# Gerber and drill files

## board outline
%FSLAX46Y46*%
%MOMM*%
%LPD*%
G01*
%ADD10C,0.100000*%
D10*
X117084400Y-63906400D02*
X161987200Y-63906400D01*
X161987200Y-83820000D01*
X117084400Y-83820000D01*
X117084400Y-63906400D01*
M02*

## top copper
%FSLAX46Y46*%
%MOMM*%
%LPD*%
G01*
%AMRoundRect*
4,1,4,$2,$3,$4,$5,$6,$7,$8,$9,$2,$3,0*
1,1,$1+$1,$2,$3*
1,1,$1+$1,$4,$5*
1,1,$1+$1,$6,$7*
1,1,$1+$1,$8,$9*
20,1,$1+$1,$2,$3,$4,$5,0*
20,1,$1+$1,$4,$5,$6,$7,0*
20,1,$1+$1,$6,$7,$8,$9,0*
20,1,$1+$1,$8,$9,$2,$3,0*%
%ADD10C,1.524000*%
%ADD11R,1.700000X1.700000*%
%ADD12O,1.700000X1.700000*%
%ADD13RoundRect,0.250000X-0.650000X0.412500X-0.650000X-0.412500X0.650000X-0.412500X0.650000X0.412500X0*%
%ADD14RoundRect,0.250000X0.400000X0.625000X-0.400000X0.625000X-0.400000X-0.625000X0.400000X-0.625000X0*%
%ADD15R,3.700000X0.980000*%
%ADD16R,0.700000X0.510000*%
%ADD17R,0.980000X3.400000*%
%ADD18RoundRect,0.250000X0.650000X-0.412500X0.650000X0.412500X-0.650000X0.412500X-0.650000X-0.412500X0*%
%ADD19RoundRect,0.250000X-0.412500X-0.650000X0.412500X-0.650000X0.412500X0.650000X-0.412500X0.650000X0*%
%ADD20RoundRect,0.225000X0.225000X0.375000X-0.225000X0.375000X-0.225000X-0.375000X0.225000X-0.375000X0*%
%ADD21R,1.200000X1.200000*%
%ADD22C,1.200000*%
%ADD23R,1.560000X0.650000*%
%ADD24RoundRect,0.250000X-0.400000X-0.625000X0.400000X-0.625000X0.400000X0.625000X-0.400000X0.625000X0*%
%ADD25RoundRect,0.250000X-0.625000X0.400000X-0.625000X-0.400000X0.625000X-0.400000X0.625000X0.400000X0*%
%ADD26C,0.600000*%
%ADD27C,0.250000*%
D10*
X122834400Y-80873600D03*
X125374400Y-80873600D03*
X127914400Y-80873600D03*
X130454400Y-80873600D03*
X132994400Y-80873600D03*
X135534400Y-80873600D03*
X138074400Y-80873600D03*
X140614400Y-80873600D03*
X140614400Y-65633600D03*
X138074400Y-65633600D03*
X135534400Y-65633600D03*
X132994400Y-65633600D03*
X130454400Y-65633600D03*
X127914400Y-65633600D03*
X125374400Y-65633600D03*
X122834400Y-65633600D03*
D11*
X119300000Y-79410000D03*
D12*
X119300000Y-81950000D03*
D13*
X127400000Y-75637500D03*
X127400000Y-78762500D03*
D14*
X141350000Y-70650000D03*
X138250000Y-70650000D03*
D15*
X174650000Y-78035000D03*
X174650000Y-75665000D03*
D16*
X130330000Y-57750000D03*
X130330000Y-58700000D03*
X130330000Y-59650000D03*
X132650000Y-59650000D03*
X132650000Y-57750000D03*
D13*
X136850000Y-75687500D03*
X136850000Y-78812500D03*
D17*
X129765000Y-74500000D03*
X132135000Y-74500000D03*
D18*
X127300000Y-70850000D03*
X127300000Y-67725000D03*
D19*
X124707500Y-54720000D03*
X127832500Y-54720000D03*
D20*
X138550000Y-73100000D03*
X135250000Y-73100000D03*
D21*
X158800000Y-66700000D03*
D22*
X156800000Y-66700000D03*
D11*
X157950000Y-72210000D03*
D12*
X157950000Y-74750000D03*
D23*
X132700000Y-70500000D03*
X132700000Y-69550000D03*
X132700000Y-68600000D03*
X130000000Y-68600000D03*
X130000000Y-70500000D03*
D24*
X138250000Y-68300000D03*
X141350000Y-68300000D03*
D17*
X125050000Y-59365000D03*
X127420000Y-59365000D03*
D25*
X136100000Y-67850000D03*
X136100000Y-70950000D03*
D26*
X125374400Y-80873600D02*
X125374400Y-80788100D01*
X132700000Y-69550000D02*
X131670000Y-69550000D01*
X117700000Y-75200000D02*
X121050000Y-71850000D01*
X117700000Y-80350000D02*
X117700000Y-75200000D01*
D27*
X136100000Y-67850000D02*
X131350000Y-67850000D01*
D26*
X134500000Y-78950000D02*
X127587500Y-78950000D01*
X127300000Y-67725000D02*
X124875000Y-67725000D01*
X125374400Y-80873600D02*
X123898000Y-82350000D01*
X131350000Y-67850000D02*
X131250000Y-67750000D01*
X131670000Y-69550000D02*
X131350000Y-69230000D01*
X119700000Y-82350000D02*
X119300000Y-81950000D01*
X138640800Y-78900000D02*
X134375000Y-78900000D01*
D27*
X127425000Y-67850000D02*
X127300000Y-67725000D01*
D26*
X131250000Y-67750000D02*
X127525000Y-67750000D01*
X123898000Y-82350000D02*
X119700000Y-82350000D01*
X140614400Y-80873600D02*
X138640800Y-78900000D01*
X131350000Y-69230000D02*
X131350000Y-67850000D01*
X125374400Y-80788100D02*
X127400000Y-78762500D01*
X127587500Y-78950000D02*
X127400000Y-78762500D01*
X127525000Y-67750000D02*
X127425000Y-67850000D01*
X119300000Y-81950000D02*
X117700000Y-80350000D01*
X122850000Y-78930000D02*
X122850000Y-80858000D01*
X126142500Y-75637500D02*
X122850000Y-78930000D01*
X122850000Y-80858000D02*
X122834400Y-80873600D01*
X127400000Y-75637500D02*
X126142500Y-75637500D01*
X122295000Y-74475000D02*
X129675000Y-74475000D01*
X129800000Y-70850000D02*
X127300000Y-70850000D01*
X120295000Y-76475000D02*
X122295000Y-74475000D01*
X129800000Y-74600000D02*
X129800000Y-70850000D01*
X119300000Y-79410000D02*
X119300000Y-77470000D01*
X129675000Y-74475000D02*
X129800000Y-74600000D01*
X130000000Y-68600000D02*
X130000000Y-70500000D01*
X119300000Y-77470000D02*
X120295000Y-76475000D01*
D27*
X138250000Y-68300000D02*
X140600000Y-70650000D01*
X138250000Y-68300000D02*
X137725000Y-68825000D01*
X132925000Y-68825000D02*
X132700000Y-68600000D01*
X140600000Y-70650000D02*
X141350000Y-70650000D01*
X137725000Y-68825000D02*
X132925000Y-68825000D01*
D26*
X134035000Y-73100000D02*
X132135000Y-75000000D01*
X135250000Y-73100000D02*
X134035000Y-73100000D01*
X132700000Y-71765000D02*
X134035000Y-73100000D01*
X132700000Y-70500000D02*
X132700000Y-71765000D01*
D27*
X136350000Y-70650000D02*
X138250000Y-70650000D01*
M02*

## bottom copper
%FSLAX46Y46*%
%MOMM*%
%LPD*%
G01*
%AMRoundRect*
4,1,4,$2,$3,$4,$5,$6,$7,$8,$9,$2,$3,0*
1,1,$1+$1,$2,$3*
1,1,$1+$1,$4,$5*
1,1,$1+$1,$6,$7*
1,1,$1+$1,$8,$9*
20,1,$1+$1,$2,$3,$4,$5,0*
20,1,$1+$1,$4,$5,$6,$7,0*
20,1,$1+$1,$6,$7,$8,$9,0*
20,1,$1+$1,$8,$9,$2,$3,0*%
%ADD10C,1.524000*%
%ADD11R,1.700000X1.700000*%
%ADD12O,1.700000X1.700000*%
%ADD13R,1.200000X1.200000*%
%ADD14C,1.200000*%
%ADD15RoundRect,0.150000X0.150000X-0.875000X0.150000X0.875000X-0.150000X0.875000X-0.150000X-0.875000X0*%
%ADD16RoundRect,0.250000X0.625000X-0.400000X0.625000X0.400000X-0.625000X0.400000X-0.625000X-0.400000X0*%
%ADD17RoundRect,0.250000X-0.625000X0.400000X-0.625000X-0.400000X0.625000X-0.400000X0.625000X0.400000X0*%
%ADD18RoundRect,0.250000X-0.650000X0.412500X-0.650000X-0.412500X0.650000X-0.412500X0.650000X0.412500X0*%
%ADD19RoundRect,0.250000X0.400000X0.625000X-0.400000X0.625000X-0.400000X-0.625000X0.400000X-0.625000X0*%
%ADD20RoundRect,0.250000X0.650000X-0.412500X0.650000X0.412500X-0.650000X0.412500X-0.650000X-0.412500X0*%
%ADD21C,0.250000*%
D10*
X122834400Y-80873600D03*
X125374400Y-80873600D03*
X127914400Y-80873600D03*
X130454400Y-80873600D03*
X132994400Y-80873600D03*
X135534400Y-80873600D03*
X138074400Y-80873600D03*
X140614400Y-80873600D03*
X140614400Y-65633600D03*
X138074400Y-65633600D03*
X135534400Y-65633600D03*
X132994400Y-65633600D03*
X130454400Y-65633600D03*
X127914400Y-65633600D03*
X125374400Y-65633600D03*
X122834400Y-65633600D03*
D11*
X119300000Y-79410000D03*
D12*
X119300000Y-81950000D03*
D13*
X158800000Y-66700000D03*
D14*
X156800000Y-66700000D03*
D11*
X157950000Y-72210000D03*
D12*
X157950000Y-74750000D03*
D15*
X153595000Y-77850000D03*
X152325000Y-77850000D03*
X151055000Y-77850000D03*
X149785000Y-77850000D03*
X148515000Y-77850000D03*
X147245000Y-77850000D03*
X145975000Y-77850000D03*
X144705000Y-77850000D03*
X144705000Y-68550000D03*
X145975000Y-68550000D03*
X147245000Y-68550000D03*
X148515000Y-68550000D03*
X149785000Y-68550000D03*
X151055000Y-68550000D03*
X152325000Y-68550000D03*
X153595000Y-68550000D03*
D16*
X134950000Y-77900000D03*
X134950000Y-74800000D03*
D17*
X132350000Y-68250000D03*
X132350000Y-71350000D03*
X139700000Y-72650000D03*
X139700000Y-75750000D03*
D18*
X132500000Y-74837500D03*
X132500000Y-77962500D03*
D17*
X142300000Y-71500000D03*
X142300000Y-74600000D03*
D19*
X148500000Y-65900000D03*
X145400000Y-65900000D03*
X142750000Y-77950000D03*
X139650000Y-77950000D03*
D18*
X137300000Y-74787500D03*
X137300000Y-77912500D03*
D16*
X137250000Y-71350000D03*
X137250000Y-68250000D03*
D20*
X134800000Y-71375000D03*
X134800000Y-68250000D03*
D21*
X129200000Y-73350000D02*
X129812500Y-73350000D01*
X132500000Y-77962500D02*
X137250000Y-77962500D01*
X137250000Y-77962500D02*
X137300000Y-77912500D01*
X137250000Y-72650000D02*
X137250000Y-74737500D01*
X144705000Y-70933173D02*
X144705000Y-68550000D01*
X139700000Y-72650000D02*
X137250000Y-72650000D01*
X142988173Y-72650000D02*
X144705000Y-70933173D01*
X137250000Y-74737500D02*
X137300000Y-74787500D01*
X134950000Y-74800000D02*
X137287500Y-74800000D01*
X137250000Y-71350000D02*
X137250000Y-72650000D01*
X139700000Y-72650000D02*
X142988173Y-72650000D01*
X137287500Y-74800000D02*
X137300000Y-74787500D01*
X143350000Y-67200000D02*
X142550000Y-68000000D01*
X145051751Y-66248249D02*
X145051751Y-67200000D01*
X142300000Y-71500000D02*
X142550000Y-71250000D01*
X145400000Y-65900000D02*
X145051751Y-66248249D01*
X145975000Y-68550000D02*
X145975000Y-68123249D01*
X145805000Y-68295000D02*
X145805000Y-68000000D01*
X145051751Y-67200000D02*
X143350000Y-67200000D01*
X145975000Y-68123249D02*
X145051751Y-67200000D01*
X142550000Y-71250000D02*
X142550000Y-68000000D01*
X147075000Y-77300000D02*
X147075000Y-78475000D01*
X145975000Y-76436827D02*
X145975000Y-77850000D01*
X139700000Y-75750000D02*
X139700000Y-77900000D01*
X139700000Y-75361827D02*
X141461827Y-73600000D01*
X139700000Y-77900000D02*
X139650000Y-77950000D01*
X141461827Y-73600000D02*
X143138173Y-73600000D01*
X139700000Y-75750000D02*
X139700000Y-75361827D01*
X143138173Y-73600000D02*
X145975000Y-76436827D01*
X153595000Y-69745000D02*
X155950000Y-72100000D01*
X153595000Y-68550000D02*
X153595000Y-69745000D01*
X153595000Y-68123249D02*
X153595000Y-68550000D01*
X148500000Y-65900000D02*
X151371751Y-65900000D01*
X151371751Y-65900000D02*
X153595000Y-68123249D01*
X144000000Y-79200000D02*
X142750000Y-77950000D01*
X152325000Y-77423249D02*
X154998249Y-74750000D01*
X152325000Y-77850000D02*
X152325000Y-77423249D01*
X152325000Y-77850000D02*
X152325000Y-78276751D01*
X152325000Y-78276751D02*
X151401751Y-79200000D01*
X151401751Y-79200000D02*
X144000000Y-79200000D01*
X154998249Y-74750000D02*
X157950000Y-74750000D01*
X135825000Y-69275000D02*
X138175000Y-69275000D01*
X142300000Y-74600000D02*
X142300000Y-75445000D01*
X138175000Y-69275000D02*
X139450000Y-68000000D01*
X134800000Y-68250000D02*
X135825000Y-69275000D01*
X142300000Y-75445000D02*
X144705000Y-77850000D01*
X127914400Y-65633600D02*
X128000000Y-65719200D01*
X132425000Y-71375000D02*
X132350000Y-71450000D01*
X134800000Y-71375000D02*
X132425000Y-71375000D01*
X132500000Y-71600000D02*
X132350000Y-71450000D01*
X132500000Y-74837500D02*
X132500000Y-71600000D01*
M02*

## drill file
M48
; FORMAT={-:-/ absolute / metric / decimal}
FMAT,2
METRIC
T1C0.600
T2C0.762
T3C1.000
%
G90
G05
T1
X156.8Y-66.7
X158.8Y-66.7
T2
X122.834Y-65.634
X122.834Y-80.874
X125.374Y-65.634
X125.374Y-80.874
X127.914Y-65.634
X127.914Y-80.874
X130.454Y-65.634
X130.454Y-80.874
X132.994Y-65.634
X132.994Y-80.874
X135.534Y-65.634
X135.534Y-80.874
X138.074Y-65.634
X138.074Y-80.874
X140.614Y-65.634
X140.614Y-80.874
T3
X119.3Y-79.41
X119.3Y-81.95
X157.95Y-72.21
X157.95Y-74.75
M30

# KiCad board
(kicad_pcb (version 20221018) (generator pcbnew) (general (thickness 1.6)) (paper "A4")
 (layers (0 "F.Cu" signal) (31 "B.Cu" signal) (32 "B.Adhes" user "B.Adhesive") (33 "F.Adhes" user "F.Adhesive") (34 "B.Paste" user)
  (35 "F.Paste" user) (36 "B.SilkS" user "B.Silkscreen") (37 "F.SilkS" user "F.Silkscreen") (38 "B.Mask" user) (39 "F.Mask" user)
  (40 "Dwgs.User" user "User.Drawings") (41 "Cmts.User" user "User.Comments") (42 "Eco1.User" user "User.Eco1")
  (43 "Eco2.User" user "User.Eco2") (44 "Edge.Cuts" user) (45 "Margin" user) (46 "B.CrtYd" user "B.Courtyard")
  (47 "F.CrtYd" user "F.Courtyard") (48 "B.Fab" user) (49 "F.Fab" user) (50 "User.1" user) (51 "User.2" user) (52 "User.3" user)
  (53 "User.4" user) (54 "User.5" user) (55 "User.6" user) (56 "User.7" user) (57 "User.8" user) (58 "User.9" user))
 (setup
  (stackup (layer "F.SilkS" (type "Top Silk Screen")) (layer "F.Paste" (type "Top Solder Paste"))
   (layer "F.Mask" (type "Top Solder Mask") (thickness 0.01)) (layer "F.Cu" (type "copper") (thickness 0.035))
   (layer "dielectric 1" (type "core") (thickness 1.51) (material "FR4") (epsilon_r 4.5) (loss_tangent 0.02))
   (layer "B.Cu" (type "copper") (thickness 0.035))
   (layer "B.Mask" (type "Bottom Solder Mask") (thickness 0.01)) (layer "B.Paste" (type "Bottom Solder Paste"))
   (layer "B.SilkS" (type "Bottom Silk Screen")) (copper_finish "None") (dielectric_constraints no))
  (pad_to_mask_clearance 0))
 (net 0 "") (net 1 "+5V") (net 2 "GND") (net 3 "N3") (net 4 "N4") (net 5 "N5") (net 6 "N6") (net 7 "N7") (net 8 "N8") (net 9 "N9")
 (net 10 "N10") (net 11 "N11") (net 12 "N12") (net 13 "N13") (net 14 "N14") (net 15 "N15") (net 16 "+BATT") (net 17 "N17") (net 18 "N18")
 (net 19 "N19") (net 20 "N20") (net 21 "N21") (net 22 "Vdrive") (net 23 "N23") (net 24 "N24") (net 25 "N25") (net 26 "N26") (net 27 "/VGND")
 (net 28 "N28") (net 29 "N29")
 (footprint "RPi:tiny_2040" (layer "F.Cu") (at 130.4544 73.2536 90)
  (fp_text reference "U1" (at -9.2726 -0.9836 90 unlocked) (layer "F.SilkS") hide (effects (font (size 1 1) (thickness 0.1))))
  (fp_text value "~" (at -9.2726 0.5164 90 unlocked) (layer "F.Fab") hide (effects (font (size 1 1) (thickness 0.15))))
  (pad "1" thru_hole circle (at -7.62 -7.62 90) (size 1.524 1.524) (drill 0.762) (layers "*.Cu" "*.Mask") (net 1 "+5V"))
  (pad "2" thru_hole circle (at -7.62 -5.08 90) (size 1.524 1.524) (drill 0.762) (layers "*.Cu" "*.Mask") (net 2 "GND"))
  (pad "3" thru_hole circle (at -7.62 -2.54 90) (size 1.524 1.524) (drill 0.762) (layers "*.Cu" "*.Mask") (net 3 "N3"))
  (pad "4" thru_hole circle (at -7.62 0 90) (size 1.524 1.524) (drill 0.762) (layers "*.Cu" "*.Mask") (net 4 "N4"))
  (pad "5" thru_hole circle (at -7.62 2.54 90) (size 1.524 1.524) (drill 0.762) (layers "*.Cu" "*.Mask") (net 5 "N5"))
  (pad "6" thru_hole circle (at -7.62 5.08 90) (size 1.524 1.524) (drill 0.762) (layers "*.Cu" "*.Mask") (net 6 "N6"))
  (pad "7" thru_hole circle (at -7.62 7.62 90) (size 1.524 1.524) (drill 0.762) (layers "*.Cu" "*.Mask") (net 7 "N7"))
  (pad "8" thru_hole circle (at -7.62 10.16 90) (size 1.524 1.524) (drill 0.762) (layers "*.Cu" "*.Mask") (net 2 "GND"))
  (pad "9" thru_hole circle (at 7.62 10.16 90) (size 1.524 1.524) (drill 0.762) (layers "*.Cu" "*.Mask") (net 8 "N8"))
  (pad "10" thru_hole circle (at 7.62 7.62 90) (size 1.524 1.524) (drill 0.762) (layers "*.Cu" "*.Mask") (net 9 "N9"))
  (pad "11" thru_hole circle (at 7.62 5.08 90) (size 1.524 1.524) (drill 0.762) (layers "*.Cu" "*.Mask") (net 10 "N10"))
  (pad "12" thru_hole circle (at 7.62 2.54 90) (size 1.524 1.524) (drill 0.762) (layers "*.Cu" "*.Mask") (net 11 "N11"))
  (pad "13" thru_hole circle (at 7.62 0 90) (size 1.524 1.524) (drill 0.762) (layers "*.Cu" "*.Mask") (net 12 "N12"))
  (pad "14" thru_hole circle (at 7.62 -2.54 90) (size 1.524 1.524) (drill 0.762) (layers "*.Cu" "*.Mask") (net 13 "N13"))
  (pad "15" thru_hole circle (at 7.62 -5.08 90) (size 1.524 1.524) (drill 0.762) (layers "*.Cu" "*.Mask") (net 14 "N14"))
  (pad "16" thru_hole circle (at 7.62 -7.62 90) (size 1.524 1.524) (drill 0.762) (layers "*.Cu" "*.Mask") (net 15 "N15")))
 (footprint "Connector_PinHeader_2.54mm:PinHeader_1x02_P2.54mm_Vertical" (layer "F.Cu") (at 119.3 79.41)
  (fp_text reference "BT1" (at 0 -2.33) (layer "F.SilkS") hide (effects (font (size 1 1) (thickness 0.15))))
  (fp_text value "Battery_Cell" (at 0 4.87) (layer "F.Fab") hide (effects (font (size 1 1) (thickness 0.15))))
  (pad "1" thru_hole rect (at 0 0) (size 1.7 1.7) (drill 1) (layers "*.Cu" "*.Mask") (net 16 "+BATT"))
  (pad "2" thru_hole oval (at 0 2.54) (size 1.7 1.7) (drill 1) (layers "*.Cu" "*.Mask") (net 2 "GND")))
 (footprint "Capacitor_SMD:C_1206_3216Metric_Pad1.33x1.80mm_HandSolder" (layer "F.Cu") (at 127.4 77.2 -90)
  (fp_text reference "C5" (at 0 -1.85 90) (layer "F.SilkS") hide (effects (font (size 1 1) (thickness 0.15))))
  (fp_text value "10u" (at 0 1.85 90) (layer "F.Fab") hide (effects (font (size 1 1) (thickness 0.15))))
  (pad "1" smd roundrect (at -1.5625 0 270) (size 1.325 1.8) (layers "F.Cu" "F.Paste" "F.Mask") (roundrect_rratio 0.188679) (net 1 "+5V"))
  (pad "2" smd roundrect (at 1.5625 0 270) (size 1.325 1.8) (layers "F.Cu" "F.Paste" "F.Mask") (roundrect_rratio 0.188679) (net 2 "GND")))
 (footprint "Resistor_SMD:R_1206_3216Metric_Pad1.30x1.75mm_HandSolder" (layer "F.Cu") (at 139.8 70.65 180)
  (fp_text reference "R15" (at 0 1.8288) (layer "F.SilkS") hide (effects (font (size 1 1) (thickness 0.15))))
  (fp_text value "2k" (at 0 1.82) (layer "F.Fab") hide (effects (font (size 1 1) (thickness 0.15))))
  (pad "1" smd roundrect (at -1.55 0 180) (size 1.3 1.75) (layers "F.Cu" "F.Paste" "F.Mask") (roundrect_rratio 0.1923076923) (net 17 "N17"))
  (pad "2" smd roundrect (at 1.55 0 180) (size 1.3 1.75) (layers "F.Cu" "F.Paste" "F.Mask") (roundrect_rratio 0.1923076923) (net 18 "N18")))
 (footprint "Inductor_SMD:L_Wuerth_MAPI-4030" (layer "F.Cu") (at 174.65 76.85 90)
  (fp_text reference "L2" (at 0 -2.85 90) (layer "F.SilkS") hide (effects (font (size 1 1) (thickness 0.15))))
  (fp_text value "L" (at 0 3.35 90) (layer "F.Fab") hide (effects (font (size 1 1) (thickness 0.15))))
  (pad "1" smd rect (at -1.185 0 90) (size 0.98 3.7) (layers "F.Cu" "F.Paste" "F.Mask") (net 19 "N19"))
  (pad "2" smd rect (at 1.185 0 90) (size 0.98 3.7) (layers "F.Cu" "F.Paste" "F.Mask") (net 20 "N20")))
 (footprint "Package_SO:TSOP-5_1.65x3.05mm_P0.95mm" (layer "F.Cu") (at 131.49 58.7)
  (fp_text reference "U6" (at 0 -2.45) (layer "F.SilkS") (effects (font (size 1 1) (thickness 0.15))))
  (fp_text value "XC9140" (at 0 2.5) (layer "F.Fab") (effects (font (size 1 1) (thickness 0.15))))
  (pad "1" smd rect (at -1.16 -0.95) (size 0.7 0.51) (layers "F.Cu" "F.Paste" "F.Mask") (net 16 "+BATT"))
  (pad "2" smd rect (at -1.16 0) (size 0.7 0.51) (layers "F.Cu" "F.Paste" "F.Mask") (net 2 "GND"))
  (pad "3" smd rect (at -1.16 0.95) (size 0.7 0.51) (layers "F.Cu" "F.Paste" "F.Mask") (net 16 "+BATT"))
  (pad "4" smd rect (at 1.16 0.95) (size 0.7 0.51) (layers "F.Cu" "F.Paste" "F.Mask") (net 1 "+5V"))
  (pad "5" smd rect (at 1.16 -0.95) (size 0.7 0.51) (layers "F.Cu" "F.Paste" "F.Mask") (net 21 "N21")))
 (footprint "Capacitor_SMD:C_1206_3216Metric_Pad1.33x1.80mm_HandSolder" (layer "F.Cu") (at 136.85 77.25 -90)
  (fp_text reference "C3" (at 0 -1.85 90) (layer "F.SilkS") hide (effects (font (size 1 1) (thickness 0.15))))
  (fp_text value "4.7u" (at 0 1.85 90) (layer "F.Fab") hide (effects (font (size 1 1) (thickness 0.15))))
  (pad "1" smd roundrect (at -1.5625 0 270) (size 1.325 1.8) (layers "F.Cu" "F.Paste" "F.Mask") (roundrect_rratio 0.1886792453)
   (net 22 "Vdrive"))
  (pad "2" smd roundrect (at 1.5625 0 270) (size 1.325 1.8) (layers "F.Cu" "F.Paste" "F.Mask") (roundrect_rratio 0.1886792453) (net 2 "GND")))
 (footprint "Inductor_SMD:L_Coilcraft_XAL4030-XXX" (layer "F.Cu") (at 130.95 74.5)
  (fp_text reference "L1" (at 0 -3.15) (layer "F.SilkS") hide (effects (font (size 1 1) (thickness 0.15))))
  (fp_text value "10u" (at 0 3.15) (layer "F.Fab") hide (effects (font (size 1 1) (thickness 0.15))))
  (pad "1" smd rect (at -1.185 0) (size 0.98 3.4) (layers "F.Cu" "F.Paste" "F.Mask") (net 16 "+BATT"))
  (pad "2" smd rect (at 1.185 0) (size 0.98 3.4) (layers "F.Cu" "F.Paste" "F.Mask") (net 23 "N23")))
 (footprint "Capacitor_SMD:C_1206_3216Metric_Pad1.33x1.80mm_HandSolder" (layer "F.Cu") (at 127.3 69.2875 90)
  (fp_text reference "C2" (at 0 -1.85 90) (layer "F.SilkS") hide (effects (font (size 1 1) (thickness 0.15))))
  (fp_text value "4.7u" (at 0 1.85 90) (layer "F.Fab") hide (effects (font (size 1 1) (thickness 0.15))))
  (pad "1" smd roundrect (at -1.5625 0 90) (size 1.325 1.8) (layers "F.Cu" "F.Paste" "F.Mask") (roundrect_rratio 0.188679) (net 16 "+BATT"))
  (pad "2" smd roundrect (at 1.5625 0 90) (size 1.325 1.8) (layers "F.Cu" "F.Paste" "F.Mask") (roundrect_rratio 0.188679) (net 2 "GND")))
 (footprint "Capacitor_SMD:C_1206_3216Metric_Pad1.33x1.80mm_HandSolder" (layer "F.Cu") (at 126.27 54.72)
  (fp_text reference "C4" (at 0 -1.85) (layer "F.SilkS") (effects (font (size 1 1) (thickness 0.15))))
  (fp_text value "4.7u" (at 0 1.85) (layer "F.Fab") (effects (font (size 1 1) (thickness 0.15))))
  (pad "1" smd roundrect (at -1.5625 0) (size 1.325 1.8) (layers "F.Cu" "F.Paste" "F.Mask") (roundrect_rratio 0.188679) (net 16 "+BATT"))
  (pad "2" smd roundrect (at 1.5625 0) (size 1.325 1.8) (layers "F.Cu" "F.Paste" "F.Mask") (roundrect_rratio 0.188679) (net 2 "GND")))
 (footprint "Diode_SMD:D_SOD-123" (layer "F.Cu") (at 136.9 73.1 180)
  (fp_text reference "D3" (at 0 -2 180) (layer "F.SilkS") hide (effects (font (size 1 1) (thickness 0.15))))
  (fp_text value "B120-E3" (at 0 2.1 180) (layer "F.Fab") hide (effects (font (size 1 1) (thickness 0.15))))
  (pad "1" smd roundrect (at -1.65 0 180) (size 0.9 1.2) (layers "F.Cu" "F.Paste" "F.Mask") (roundrect_rratio 0.25) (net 22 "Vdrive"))
  (pad "2" smd roundrect (at 1.65 0 180) (size 0.9 1.2) (layers "F.Cu" "F.Paste" "F.Mask") (roundrect_rratio 0.25) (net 23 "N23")))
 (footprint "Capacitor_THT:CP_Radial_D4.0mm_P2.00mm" (layer "F.Cu") (at 158.8 66.7 180)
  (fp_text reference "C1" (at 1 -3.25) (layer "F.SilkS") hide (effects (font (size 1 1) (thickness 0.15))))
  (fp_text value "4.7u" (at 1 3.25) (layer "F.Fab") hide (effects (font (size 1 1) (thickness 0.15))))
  (pad "1" thru_hole rect (at 0 0 180) (size 1.2 1.2) (drill 0.6) (layers "*.Cu" "*.Mask") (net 22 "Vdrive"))
  (pad "2" thru_hole circle (at 2 0 180) (size 1.2 1.2) (drill 0.6) (layers "*.Cu" "*.Mask") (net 2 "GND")))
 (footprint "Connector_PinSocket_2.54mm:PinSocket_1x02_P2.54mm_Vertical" (layer "F.Cu") (at 157.95 72.21)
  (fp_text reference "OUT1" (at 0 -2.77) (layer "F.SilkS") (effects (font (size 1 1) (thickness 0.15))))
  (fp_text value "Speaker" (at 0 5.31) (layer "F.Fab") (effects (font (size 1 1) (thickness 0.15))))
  (pad "1" thru_hole rect (at 0 0) (size 1.7 1.7) (drill 1) (layers "*.Cu" "*.Mask") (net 20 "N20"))
  (pad "2" thru_hole oval (at 0 2.54) (size 1.7 1.7) (drill 1) (layers "*.Cu" "*.Mask") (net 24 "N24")))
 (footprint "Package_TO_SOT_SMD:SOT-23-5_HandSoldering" (layer "F.Cu") (at 131.35 69.55 180)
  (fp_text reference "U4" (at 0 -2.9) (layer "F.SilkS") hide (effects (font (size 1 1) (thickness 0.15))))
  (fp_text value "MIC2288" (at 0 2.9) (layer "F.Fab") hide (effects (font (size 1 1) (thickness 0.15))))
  (pad "1" smd rect (at -1.35 -0.95 180) (size 1.56 0.65) (layers "F.Cu" "F.Paste" "F.Mask") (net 23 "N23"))
  (pad "2" smd rect (at -1.35 0 180) (size 1.56 0.65) (layers "F.Cu" "F.Paste" "F.Mask") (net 2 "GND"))
  (pad "3" smd rect (at -1.35 0.95 180) (size 1.56 0.65) (layers "F.Cu" "F.Paste" "F.Mask") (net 17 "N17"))
  (pad "4" smd rect (at 1.35 0.95 180) (size 1.56 0.65) (layers "F.Cu" "F.Paste" "F.Mask") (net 16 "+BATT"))
  (pad "5" smd rect (at 1.35 -0.95 180) (size 1.56 0.65) (layers "F.Cu" "F.Paste" "F.Mask") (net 16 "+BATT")))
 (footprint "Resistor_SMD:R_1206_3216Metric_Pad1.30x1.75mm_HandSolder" (layer "F.Cu") (at 139.8 68.3)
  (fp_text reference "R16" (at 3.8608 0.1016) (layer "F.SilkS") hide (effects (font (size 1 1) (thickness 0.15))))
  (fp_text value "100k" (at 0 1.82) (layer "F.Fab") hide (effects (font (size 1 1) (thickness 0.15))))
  (pad "1" smd roundrect (at -1.55 0) (size 1.3 1.75) (layers "F.Cu" "F.Paste" "F.Mask") (roundrect_rratio 0.1923076923) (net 17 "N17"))
  (pad "2" smd roundrect (at 1.55 0) (size 1.3 1.75) (layers "F.Cu" "F.Paste" "F.Mask") (roundrect_rratio 0.1923076923) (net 22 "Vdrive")))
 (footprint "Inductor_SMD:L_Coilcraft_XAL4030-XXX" (layer "F.Cu") (at 126.235 59.365)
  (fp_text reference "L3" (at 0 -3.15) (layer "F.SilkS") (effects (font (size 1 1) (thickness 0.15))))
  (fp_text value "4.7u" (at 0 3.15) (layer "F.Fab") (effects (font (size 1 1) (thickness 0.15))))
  (pad "1" smd rect (at -1.185 0) (size 0.98 3.4) (layers "F.Cu" "F.Paste" "F.Mask") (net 16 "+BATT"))
  (pad "2" smd rect (at 1.185 0) (size 0.98 3.4) (layers "F.Cu" "F.Paste" "F.Mask") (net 21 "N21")))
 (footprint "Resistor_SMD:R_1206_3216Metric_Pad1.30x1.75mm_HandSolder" (layer "F.Cu") (at 136.1 69.4 -90)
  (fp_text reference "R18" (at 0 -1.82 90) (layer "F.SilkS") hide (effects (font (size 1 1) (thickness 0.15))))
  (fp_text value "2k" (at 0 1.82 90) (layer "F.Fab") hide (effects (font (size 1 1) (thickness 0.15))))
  (pad "1" smd roundrect (at -1.55 0 270) (size 1.3 1.75) (layers "F.Cu" "F.Paste" "F.Mask") (roundrect_rratio 0.1923076923) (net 2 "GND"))
  (pad "2" smd roundrect (at 1.55 0 270) (size 1.3 1.75) (layers "F.Cu" "F.Paste" "F.Mask") (roundrect_rratio 0.1923076923) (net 18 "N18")))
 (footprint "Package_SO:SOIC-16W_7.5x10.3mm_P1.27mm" (layer "B.Cu") (at 149.15 73.2 90)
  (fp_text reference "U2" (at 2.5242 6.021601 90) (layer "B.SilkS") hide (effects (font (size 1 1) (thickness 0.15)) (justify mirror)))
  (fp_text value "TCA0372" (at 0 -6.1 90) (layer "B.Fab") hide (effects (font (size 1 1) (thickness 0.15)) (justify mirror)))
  (pad "1" smd roundrect (at -4.65 4.445 90) (size 2.05 0.6) (layers "B.Cu" "B.Paste" "B.Mask") (roundrect_rratio 0.25) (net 22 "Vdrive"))
  (pad "2" smd roundrect (at -4.65 3.175 90) (size 2.05 0.6) (layers "B.Cu" "B.Paste" "B.Mask") (roundrect_rratio 0.25) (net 24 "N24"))
  (pad "3" smd roundrect (at -4.65 1.905 90) (size 2.05 0.6) (layers "B.Cu" "B.Paste" "B.Mask") (roundrect_rratio 0.25))
  (pad "4" smd roundrect (at -4.65 0.635 90) (size 2.05 0.6) (layers "B.Cu" "B.Paste" "B.Mask") (roundrect_rratio 0.25) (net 2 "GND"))
  (pad "5" smd roundrect (at -4.65 -0.635 90) (size 2.05 0.6) (layers "B.Cu" "B.Paste" "B.Mask") (roundrect_rratio 0.25) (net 2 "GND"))
  (pad "6" smd roundrect (at -4.65 -1.905 90) (size 2.05 0.6) (layers "B.Cu" "B.Paste" "B.Mask") (roundrect_rratio 0.25))
  (pad "7" smd roundrect (at -4.65 -3.175 90) (size 2.05 0.6) (layers "B.Cu" "B.Paste" "B.Mask") (roundrect_rratio 0.25) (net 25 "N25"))
  (pad "8" smd roundrect (at -4.65 -4.445 90) (size 2.05 0.6) (layers "B.Cu" "B.Paste" "B.Mask") (roundrect_rratio 0.25) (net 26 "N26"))
  (pad "9" smd roundrect (at 4.65 -4.445 90) (size 2.05 0.6) (layers "B.Cu" "B.Paste" "B.Mask") (roundrect_rratio 0.25) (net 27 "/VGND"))
  (pad "10" smd roundrect (at 4.65 -3.175 90) (size 2.05 0.6) (layers "B.Cu" "B.Paste" "B.Mask") (roundrect_rratio 0.25) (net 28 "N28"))
  (pad "11" smd roundrect (at 4.65 -1.905 90) (size 2.05 0.6) (layers "B.Cu" "B.Paste" "B.Mask") (roundrect_rratio 0.25))
  (pad "12" smd roundrect (at 4.65 -0.635 90) (size 2.05 0.6) (layers "B.Cu" "B.Paste" "B.Mask") (roundrect_rratio 0.25) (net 2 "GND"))
  (pad "13" smd roundrect (at 4.65 0.635 90) (size 2.05 0.6) (layers "B.Cu" "B.Paste" "B.Mask") (roundrect_rratio 0.25) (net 2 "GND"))
  (pad "14" smd roundrect (at 4.65 1.905 90) (size 2.05 0.6) (layers "B.Cu" "B.Paste" "B.Mask") (roundrect_rratio 0.25))
  (pad "15" smd roundrect (at 4.65 3.175 90) (size 2.05 0.6) (layers "B.Cu" "B.Paste" "B.Mask") (roundrect_rratio 0.25))
  (pad "16" smd roundrect (at 4.65 4.445 90) (size 2.05 0.6) (layers "B.Cu" "B.Paste" "B.Mask") (roundrect_rratio 0.25) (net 19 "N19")))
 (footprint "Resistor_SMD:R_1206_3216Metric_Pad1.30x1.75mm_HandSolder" (layer "B.Cu") (at 134.95 76.35 90)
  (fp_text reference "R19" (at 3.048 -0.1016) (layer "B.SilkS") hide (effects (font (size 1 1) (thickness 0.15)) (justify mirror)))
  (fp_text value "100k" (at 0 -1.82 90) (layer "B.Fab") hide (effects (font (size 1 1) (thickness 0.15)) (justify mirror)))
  (pad "1" smd roundrect (at -1.55 0 90) (size 1.3 1.75) (layers "B.Cu" "B.Paste" "B.Mask") (roundrect_rratio 0.1923076923) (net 2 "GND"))
  (pad "2" smd roundrect (at 1.55 0 90) (size 1.3 1.75) (layers "B.Cu" "B.Paste" "B.Mask") (roundrect_rratio 0.1923076923) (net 27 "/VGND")))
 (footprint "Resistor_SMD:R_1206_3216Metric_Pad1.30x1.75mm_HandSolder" (layer "B.Cu") (at 132.35 69.8 -90)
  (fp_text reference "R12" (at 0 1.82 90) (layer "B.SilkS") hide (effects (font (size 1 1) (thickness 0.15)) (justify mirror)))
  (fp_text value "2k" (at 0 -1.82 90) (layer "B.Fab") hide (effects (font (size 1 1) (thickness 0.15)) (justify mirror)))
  (pad "1" smd roundrect (at -1.55 0 270) (size 1.3 1.75) (layers "B.Cu" "B.Paste" "B.Mask") (roundrect_rratio 0.1923076923) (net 14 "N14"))
  (pad "2" smd roundrect (at 1.55 0 270) (size 1.3 1.75) (layers "B.Cu" "B.Paste" "B.Mask") (roundrect_rratio 0.1923076923) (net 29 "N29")))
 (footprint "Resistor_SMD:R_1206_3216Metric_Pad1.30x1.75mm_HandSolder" (layer "B.Cu") (at 139.7 74.2 -90)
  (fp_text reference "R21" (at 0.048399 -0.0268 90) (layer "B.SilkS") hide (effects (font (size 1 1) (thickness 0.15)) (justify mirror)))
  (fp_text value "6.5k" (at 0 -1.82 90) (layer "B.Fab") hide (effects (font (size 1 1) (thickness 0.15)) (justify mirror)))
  (pad "1" smd roundrect (at -1.55 0 270) (size 1.3 1.75) (layers "B.Cu" "B.Paste" "B.Mask") (roundrect_rratio 0.1923076923)
   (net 27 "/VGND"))
  (pad "2" smd roundrect (at 1.55 0 270) (size 1.3 1.75) (layers "B.Cu" "B.Paste" "B.Mask") (roundrect_rratio 0.1923076923) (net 25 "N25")))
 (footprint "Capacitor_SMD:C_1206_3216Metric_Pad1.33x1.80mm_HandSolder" (layer "B.Cu") (at 132.5 76.4 -90)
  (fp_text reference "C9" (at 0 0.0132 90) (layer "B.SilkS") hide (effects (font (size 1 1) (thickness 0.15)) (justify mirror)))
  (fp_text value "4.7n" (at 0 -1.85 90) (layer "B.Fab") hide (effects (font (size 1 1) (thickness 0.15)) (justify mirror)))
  (pad "1" smd roundrect (at -1.5625 0 270) (size 1.325 1.8) (layers "B.Cu" "B.Paste" "B.Mask") (roundrect_rratio 0.1886792453)
   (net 29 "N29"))
  (pad "2" smd roundrect (at 1.5625 0 270) (size 1.325 1.8) (layers "B.Cu" "B.Paste" "B.Mask") (roundrect_rratio 0.1886792453) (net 2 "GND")))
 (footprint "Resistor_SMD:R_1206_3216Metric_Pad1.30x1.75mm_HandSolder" (layer "B.Cu") (at 142.3 73.05 -90)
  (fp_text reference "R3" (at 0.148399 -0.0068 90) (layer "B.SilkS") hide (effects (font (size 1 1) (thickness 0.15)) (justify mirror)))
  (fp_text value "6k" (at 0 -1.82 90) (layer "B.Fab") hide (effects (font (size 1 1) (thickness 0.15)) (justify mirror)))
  (pad "1" smd roundrect (at -1.55 0 270) (size 1.3 1.75) (layers "B.Cu" "B.Paste" "B.Mask") (roundrect_rratio 0.1923076923) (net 28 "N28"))
  (pad "2" smd roundrect (at 1.55 0 270) (size 1.3 1.75) (layers "B.Cu" "B.Paste" "B.Mask") (roundrect_rratio 0.1923076923) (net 26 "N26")))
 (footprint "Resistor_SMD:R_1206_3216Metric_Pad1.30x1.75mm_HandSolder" (layer "B.Cu") (at 146.95 65.9 180)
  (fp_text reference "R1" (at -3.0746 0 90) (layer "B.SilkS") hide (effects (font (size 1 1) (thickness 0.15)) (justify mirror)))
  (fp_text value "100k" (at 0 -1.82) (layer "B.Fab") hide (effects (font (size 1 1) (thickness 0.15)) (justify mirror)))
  (pad "1" smd roundrect (at -1.55 0 180) (size 1.3 1.75) (layers "B.Cu" "B.Paste" "B.Mask") (roundrect_rratio 0.1923076923) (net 19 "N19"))
  (pad "2" smd roundrect (at 1.55 0 180) (size 1.3 1.75) (layers "B.Cu" "B.Paste" "B.Mask") (roundrect_rratio 0.1923076923) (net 28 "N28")))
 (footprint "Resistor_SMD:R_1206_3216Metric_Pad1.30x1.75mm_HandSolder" (layer "B.Cu") (at 141.2 77.95 180)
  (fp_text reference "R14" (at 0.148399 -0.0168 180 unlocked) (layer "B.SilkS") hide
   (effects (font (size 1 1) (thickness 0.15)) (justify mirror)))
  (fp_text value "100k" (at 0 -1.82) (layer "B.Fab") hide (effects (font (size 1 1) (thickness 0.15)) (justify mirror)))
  (pad "1" smd roundrect (at -1.55 0 180) (size 1.3 1.75) (layers "B.Cu" "B.Paste" "B.Mask") (roundrect_rratio 0.1923076923) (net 24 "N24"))
  (pad "2" smd roundrect (at 1.55 0 180) (size 1.3 1.75) (layers "B.Cu" "B.Paste" "B.Mask") (roundrect_rratio 0.1923076923) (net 25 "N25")))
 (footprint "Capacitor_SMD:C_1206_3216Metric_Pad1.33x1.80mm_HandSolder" (layer "B.Cu") (at 137.3 76.35 -90)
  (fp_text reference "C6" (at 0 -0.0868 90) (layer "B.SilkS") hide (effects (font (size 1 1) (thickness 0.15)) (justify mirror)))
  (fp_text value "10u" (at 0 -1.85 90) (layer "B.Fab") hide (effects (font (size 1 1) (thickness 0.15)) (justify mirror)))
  (pad "1" smd roundrect (at -1.5625 0 270) (size 1.325 1.8) (layers "B.Cu" "B.Paste" "B.Mask") (roundrect_rratio 0.1886792453)
   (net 27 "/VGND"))
  (pad "2" smd roundrect (at 1.5625 0 270) (size 1.325 1.8) (layers "B.Cu" "B.Paste" "B.Mask") (roundrect_rratio 0.1886792453) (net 2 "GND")))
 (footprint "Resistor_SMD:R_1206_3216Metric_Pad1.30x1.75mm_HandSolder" (layer "B.Cu") (at 137.25 69.8 90)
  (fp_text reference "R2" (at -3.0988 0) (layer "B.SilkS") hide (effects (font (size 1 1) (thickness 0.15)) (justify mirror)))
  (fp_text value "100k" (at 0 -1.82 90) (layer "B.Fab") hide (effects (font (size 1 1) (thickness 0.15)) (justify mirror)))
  (pad "1" smd roundrect (at -1.55 0 90) (size 1.3 1.75) (layers "B.Cu" "B.Paste" "B.Mask") (roundrect_rratio 0.1923076923) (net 27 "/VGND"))
  (pad "2" smd roundrect (at 1.55 0 90) (size 1.3 1.75) (layers "B.Cu" "B.Paste" "B.Mask") (roundrect_rratio 0.1923076923) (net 22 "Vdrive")))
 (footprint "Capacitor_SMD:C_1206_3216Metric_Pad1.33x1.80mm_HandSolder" (layer "B.Cu") (at 134.8 69.8125 90)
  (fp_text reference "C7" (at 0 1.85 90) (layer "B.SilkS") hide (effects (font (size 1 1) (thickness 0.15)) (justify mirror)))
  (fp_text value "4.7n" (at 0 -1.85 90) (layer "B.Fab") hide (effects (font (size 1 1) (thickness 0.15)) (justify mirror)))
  (pad "1" smd roundrect (at -1.5625 0 90) (size 1.325 1.8) (layers "B.Cu" "B.Paste" "B.Mask") (roundrect_rratio 0.188679) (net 29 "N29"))
  (pad "2" smd roundrect (at 1.5625 0 90) (size 1.325 1.8) (layers "B.Cu" "B.Paste" "B.Mask") (roundrect_rratio 0.188679) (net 26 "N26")))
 (gr_rect (start 117.0844 63.9064) (end 161.9872 83.82) (stroke (width 0.1) (type default)) (fill none) (layer "Edge.Cuts"))
 (segment (start 129.2 73.35) (end 129.8125 73.35) (width 0.25) (layer "B.Cu") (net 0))
 (segment (start 125.3744 80.8736) (end 125.3744 80.7881) (width 0.6) (layer "F.Cu") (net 2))
 (segment (start 132.7 69.55) (end 131.67 69.55) (width 0.6) (layer "F.Cu") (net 2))
 (segment (start 117.7 75.2) (end 121.05 71.85) (width 0.6) (layer "F.Cu") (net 2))
 (segment (start 117.7 80.35) (end 117.7 75.2) (width 0.6) (layer "F.Cu") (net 2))
 (segment (start 136.1 67.85) (end 131.35 67.85) (width 0.25) (layer "F.Cu") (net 2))
 (segment (start 134.5 78.95) (end 127.5875 78.95) (width 0.6) (layer "F.Cu") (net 2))
 (segment (start 127.3 67.725) (end 124.875 67.725) (width 0.6) (layer "F.Cu") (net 2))
 (segment (start 125.3744 80.8736) (end 123.898 82.35) (width 0.6) (layer "F.Cu") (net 2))
 (segment (start 131.35 67.85) (end 131.25 67.75) (width 0.6) (layer "F.Cu") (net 2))
 (segment (start 131.67 69.55) (end 131.35 69.23) (width 0.6) (layer "F.Cu") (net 2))
 (segment (start 119.7 82.35) (end 119.3 81.95) (width 0.6) (layer "F.Cu") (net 2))
 (segment (start 138.6408 78.9) (end 134.375 78.9) (width 0.6) (layer "F.Cu") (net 2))
 (segment (start 127.425 67.85) (end 127.3 67.725) (width 0.25) (layer "F.Cu") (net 2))
 (segment (start 131.25 67.75) (end 127.525 67.75) (width 0.6) (layer "F.Cu") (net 2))
 (segment (start 123.898 82.35) (end 119.7 82.35) (width 0.6) (layer "F.Cu") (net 2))
 (segment (start 140.6144 80.8736) (end 138.6408 78.9) (width 0.6) (layer "F.Cu") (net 2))
 (segment (start 131.35 69.23) (end 131.35 67.85) (width 0.6) (layer "F.Cu") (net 2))
 (segment (start 125.3744 80.7881) (end 127.4 78.7625) (width 0.6) (layer "F.Cu") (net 2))
 (segment (start 127.5875 78.95) (end 127.4 78.7625) (width 0.6) (layer "F.Cu") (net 2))
 (segment (start 127.525 67.75) (end 127.425 67.85) (width 0.6) (layer "F.Cu") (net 2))
 (segment (start 119.3 81.95) (end 117.7 80.35) (width 0.6) (layer "F.Cu") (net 2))
 (segment (start 132.5 77.9625) (end 137.25 77.9625) (width 0.25) (layer "B.Cu") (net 2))
 (segment (start 137.25 77.9625) (end 137.3 77.9125) (width 0.25) (layer "B.Cu") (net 2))
 (segment (start 122.85 78.93) (end 122.85 80.858) (width 0.6) (layer "F.Cu") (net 1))
 (segment (start 126.1425 75.6375) (end 122.85 78.93) (width 0.6) (layer "F.Cu") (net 1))
 (segment (start 122.85 80.858) (end 122.8344 80.8736) (width 0.6) (layer "F.Cu") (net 1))
 (segment (start 127.4 75.6375) (end 126.1425 75.6375) (width 0.6) (layer "F.Cu") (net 1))
 (segment (start 122.295 74.475) (end 129.675 74.475) (width 0.6) (layer "F.Cu") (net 16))
 (segment (start 129.8 70.85) (end 127.3 70.85) (width 0.6) (layer "F.Cu") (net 16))
 (segment (start 120.295 76.475) (end 122.295 74.475) (width 0.6) (layer "F.Cu") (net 16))
 (segment (start 129.8 74.6) (end 129.8 70.85) (width 0.6) (layer "F.Cu") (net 16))
 (segment (start 119.3 79.41) (end 119.3 77.47) (width 0.6) (layer "F.Cu") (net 16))
 (segment (start 129.675 74.475) (end 129.8 74.6) (width 0.6) (layer "F.Cu") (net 16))
 (segment (start 130 68.6) (end 130 70.5) (width 0.6) (layer "F.Cu") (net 16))
 (segment (start 119.3 77.47) (end 120.295 76.475) (width 0.6) (layer "F.Cu") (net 16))
 (segment (start 138.25 68.3) (end 140.6 70.65) (width 0.25) (layer "F.Cu") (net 17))
 (segment (start 138.25 68.3) (end 137.725 68.825) (width 0.25) (layer "F.Cu") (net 17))
 (segment (start 132.925 68.825) (end 132.7 68.6) (width 0.25) (layer "F.Cu") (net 17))
 (segment (start 140.6 70.65) (end 141.35 70.65) (width 0.25) (layer "F.Cu") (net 17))
 (segment (start 137.725 68.825) (end 132.925 68.825) (width 0.25) (layer "F.Cu") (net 17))
 (segment (start 137.25 72.65) (end 137.25 74.7375) (width 0.25) (layer "B.Cu") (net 27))
 (segment (start 144.705 70.933173) (end 144.705 68.55) (width 0.25) (layer "B.Cu") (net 27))
 (segment (start 139.7 72.65) (end 137.25 72.65) (width 0.25) (layer "B.Cu") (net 27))
 (segment (start 142.988173 72.65) (end 144.705 70.933173) (width 0.25) (layer "B.Cu") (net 27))
 (segment (start 137.25 74.7375) (end 137.3 74.7875) (width 0.25) (layer "B.Cu") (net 27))
 (segment (start 134.95 74.8) (end 137.2875 74.8) (width 0.25) (layer "B.Cu") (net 27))
 (segment (start 137.25 71.35) (end 137.25 72.65) (width 0.25) (layer "B.Cu") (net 27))
 (segment (start 139.7 72.65) (end 142.988173 72.65) (width 0.25) (layer "B.Cu") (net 27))
 (segment (start 137.2875 74.8) (end 137.3 74.7875) (width 0.25) (layer "B.Cu") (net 27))
 (segment (start 143.35 67.2) (end 142.55 68) (width 0.25) (layer "B.Cu") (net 28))
 (segment (start 145.051751 66.248249) (end 145.051751 67.2) (width 0.25) (layer "B.Cu") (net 28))
 (segment (start 142.3 71.5) (end 142.55 71.25) (width 0.25) (layer "B.Cu") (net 28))
 (segment (start 145.4 65.9) (end 145.051751 66.248249) (width 0.25) (layer "B.Cu") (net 28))
 (segment (start 145.975 68.55) (end 145.975 68.123249) (width 0.25) (layer "B.Cu") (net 28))
 (segment (start 145.805 68.295) (end 145.805 68) (width 0.25) (layer "B.Cu") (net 28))
 (segment (start 145.051751 67.2) (end 143.35 67.2) (width 0.25) (layer "B.Cu") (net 28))
 (segment (start 145.975 68.123249) (end 145.051751 67.2) (width 0.25) (layer "B.Cu") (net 28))
 (segment (start 142.55 71.25) (end 142.55 68) (width 0.25) (layer "B.Cu") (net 28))
 (segment (start 147.075 77.3) (end 147.075 78.475) (width 0.25) (layer "B.Cu") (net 25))
 (segment (start 145.975 76.436827) (end 145.975 77.85) (width 0.25) (layer "B.Cu") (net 25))
 (segment (start 139.7 75.75) (end 139.7 77.9) (width 0.25) (layer "B.Cu") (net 25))
 (segment (start 139.7 75.361827) (end 141.461827 73.6) (width 0.25) (layer "B.Cu") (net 25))
 (segment (start 139.7 77.9) (end 139.65 77.95) (width 0.25) (layer "B.Cu") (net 25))
 (segment (start 141.461827 73.6) (end 143.138173 73.6) (width 0.25) (layer "B.Cu") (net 25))
 (segment (start 139.7 75.75) (end 139.7 75.361827) (width 0.25) (layer "B.Cu") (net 25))
 (segment (start 143.138173 73.6) (end 145.975 76.436827) (width 0.25) (layer "B.Cu") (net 25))
 (segment (start 153.595 69.745) (end 155.95 72.1) (width 0.25) (layer "B.Cu") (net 19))
 (segment (start 153.595 68.55) (end 153.595 69.745) (width 0.25) (layer "B.Cu") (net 19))
 (segment (start 153.595 68.123249) (end 153.595 68.55) (width 0.25) (layer "B.Cu") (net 19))
 (segment (start 148.5 65.9) (end 151.371751 65.9) (width 0.25) (layer "B.Cu") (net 19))
 (segment (start 151.371751 65.9) (end 153.595 68.123249) (width 0.25) (layer "B.Cu") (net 19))
 (segment (start 144 79.2) (end 142.75 77.95) (width 0.25) (layer "B.Cu") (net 24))
 (segment (start 152.325 77.423249) (end 154.998249 74.75) (width 0.25) (layer "B.Cu") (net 24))
 (segment (start 152.325 77.85) (end 152.325 77.423249) (width 0.25) (layer "B.Cu") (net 24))
 (segment (start 152.325 77.85) (end 152.325 78.276751) (width 0.25) (layer "B.Cu") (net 24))
 (segment (start 152.325 78.276751) (end 151.401751 79.2) (width 0.25) (layer "B.Cu") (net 24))
 (segment (start 151.401751 79.2) (end 144 79.2) (width 0.25) (layer "B.Cu") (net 24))
 (segment (start 154.998249 74.75) (end 157.95 74.75) (width 0.25) (layer "B.Cu") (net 24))
 (segment (start 135.825 69.275) (end 138.175 69.275) (width 0.25) (layer "B.Cu") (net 26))
 (segment (start 142.3 74.6) (end 142.3 75.445) (width 0.25) (layer "B.Cu") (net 26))
 (segment (start 138.175 69.275) (end 139.45 68) (width 0.25) (layer "B.Cu") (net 26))
 (segment (start 134.8 68.25) (end 135.825 69.275) (width 0.25) (layer "B.Cu") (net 26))
 (segment (start 142.3 75.445) (end 144.705 77.85) (width 0.25) (layer "B.Cu") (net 26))
 (segment (start 134.035 73.1) (end 132.135 75) (width 0.6) (layer "F.Cu") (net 23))
 (segment (start 135.25 73.1) (end 134.035 73.1) (width 0.6) (layer "F.Cu") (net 23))
 (segment (start 132.7 71.765) (end 134.035 73.1) (width 0.6) (layer "F.Cu") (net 23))
 (segment (start 132.7 70.5) (end 132.7 71.765) (width 0.6) (layer "F.Cu") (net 23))
 (segment (start 127.9144 65.6336) (end 128 65.7192) (width 0.25) (layer "B.Cu") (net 13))
 (segment (start 136.35 70.65) (end 138.25 70.65) (width 0.25) (layer "F.Cu") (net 18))
 (segment (start 132.425 71.375) (end 132.35 71.45) (width 0.25) (layer "B.Cu") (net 29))
 (segment (start 134.8 71.375) (end 132.425 71.375) (width 0.25) (layer "B.Cu") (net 29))
 (segment (start 132.5 71.6) (end 132.35 71.45) (width 0.25) (layer "B.Cu") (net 29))
 (segment (start 132.5 74.8375) (end 132.5 71.6) (width 0.25) (layer "B.Cu") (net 29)))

